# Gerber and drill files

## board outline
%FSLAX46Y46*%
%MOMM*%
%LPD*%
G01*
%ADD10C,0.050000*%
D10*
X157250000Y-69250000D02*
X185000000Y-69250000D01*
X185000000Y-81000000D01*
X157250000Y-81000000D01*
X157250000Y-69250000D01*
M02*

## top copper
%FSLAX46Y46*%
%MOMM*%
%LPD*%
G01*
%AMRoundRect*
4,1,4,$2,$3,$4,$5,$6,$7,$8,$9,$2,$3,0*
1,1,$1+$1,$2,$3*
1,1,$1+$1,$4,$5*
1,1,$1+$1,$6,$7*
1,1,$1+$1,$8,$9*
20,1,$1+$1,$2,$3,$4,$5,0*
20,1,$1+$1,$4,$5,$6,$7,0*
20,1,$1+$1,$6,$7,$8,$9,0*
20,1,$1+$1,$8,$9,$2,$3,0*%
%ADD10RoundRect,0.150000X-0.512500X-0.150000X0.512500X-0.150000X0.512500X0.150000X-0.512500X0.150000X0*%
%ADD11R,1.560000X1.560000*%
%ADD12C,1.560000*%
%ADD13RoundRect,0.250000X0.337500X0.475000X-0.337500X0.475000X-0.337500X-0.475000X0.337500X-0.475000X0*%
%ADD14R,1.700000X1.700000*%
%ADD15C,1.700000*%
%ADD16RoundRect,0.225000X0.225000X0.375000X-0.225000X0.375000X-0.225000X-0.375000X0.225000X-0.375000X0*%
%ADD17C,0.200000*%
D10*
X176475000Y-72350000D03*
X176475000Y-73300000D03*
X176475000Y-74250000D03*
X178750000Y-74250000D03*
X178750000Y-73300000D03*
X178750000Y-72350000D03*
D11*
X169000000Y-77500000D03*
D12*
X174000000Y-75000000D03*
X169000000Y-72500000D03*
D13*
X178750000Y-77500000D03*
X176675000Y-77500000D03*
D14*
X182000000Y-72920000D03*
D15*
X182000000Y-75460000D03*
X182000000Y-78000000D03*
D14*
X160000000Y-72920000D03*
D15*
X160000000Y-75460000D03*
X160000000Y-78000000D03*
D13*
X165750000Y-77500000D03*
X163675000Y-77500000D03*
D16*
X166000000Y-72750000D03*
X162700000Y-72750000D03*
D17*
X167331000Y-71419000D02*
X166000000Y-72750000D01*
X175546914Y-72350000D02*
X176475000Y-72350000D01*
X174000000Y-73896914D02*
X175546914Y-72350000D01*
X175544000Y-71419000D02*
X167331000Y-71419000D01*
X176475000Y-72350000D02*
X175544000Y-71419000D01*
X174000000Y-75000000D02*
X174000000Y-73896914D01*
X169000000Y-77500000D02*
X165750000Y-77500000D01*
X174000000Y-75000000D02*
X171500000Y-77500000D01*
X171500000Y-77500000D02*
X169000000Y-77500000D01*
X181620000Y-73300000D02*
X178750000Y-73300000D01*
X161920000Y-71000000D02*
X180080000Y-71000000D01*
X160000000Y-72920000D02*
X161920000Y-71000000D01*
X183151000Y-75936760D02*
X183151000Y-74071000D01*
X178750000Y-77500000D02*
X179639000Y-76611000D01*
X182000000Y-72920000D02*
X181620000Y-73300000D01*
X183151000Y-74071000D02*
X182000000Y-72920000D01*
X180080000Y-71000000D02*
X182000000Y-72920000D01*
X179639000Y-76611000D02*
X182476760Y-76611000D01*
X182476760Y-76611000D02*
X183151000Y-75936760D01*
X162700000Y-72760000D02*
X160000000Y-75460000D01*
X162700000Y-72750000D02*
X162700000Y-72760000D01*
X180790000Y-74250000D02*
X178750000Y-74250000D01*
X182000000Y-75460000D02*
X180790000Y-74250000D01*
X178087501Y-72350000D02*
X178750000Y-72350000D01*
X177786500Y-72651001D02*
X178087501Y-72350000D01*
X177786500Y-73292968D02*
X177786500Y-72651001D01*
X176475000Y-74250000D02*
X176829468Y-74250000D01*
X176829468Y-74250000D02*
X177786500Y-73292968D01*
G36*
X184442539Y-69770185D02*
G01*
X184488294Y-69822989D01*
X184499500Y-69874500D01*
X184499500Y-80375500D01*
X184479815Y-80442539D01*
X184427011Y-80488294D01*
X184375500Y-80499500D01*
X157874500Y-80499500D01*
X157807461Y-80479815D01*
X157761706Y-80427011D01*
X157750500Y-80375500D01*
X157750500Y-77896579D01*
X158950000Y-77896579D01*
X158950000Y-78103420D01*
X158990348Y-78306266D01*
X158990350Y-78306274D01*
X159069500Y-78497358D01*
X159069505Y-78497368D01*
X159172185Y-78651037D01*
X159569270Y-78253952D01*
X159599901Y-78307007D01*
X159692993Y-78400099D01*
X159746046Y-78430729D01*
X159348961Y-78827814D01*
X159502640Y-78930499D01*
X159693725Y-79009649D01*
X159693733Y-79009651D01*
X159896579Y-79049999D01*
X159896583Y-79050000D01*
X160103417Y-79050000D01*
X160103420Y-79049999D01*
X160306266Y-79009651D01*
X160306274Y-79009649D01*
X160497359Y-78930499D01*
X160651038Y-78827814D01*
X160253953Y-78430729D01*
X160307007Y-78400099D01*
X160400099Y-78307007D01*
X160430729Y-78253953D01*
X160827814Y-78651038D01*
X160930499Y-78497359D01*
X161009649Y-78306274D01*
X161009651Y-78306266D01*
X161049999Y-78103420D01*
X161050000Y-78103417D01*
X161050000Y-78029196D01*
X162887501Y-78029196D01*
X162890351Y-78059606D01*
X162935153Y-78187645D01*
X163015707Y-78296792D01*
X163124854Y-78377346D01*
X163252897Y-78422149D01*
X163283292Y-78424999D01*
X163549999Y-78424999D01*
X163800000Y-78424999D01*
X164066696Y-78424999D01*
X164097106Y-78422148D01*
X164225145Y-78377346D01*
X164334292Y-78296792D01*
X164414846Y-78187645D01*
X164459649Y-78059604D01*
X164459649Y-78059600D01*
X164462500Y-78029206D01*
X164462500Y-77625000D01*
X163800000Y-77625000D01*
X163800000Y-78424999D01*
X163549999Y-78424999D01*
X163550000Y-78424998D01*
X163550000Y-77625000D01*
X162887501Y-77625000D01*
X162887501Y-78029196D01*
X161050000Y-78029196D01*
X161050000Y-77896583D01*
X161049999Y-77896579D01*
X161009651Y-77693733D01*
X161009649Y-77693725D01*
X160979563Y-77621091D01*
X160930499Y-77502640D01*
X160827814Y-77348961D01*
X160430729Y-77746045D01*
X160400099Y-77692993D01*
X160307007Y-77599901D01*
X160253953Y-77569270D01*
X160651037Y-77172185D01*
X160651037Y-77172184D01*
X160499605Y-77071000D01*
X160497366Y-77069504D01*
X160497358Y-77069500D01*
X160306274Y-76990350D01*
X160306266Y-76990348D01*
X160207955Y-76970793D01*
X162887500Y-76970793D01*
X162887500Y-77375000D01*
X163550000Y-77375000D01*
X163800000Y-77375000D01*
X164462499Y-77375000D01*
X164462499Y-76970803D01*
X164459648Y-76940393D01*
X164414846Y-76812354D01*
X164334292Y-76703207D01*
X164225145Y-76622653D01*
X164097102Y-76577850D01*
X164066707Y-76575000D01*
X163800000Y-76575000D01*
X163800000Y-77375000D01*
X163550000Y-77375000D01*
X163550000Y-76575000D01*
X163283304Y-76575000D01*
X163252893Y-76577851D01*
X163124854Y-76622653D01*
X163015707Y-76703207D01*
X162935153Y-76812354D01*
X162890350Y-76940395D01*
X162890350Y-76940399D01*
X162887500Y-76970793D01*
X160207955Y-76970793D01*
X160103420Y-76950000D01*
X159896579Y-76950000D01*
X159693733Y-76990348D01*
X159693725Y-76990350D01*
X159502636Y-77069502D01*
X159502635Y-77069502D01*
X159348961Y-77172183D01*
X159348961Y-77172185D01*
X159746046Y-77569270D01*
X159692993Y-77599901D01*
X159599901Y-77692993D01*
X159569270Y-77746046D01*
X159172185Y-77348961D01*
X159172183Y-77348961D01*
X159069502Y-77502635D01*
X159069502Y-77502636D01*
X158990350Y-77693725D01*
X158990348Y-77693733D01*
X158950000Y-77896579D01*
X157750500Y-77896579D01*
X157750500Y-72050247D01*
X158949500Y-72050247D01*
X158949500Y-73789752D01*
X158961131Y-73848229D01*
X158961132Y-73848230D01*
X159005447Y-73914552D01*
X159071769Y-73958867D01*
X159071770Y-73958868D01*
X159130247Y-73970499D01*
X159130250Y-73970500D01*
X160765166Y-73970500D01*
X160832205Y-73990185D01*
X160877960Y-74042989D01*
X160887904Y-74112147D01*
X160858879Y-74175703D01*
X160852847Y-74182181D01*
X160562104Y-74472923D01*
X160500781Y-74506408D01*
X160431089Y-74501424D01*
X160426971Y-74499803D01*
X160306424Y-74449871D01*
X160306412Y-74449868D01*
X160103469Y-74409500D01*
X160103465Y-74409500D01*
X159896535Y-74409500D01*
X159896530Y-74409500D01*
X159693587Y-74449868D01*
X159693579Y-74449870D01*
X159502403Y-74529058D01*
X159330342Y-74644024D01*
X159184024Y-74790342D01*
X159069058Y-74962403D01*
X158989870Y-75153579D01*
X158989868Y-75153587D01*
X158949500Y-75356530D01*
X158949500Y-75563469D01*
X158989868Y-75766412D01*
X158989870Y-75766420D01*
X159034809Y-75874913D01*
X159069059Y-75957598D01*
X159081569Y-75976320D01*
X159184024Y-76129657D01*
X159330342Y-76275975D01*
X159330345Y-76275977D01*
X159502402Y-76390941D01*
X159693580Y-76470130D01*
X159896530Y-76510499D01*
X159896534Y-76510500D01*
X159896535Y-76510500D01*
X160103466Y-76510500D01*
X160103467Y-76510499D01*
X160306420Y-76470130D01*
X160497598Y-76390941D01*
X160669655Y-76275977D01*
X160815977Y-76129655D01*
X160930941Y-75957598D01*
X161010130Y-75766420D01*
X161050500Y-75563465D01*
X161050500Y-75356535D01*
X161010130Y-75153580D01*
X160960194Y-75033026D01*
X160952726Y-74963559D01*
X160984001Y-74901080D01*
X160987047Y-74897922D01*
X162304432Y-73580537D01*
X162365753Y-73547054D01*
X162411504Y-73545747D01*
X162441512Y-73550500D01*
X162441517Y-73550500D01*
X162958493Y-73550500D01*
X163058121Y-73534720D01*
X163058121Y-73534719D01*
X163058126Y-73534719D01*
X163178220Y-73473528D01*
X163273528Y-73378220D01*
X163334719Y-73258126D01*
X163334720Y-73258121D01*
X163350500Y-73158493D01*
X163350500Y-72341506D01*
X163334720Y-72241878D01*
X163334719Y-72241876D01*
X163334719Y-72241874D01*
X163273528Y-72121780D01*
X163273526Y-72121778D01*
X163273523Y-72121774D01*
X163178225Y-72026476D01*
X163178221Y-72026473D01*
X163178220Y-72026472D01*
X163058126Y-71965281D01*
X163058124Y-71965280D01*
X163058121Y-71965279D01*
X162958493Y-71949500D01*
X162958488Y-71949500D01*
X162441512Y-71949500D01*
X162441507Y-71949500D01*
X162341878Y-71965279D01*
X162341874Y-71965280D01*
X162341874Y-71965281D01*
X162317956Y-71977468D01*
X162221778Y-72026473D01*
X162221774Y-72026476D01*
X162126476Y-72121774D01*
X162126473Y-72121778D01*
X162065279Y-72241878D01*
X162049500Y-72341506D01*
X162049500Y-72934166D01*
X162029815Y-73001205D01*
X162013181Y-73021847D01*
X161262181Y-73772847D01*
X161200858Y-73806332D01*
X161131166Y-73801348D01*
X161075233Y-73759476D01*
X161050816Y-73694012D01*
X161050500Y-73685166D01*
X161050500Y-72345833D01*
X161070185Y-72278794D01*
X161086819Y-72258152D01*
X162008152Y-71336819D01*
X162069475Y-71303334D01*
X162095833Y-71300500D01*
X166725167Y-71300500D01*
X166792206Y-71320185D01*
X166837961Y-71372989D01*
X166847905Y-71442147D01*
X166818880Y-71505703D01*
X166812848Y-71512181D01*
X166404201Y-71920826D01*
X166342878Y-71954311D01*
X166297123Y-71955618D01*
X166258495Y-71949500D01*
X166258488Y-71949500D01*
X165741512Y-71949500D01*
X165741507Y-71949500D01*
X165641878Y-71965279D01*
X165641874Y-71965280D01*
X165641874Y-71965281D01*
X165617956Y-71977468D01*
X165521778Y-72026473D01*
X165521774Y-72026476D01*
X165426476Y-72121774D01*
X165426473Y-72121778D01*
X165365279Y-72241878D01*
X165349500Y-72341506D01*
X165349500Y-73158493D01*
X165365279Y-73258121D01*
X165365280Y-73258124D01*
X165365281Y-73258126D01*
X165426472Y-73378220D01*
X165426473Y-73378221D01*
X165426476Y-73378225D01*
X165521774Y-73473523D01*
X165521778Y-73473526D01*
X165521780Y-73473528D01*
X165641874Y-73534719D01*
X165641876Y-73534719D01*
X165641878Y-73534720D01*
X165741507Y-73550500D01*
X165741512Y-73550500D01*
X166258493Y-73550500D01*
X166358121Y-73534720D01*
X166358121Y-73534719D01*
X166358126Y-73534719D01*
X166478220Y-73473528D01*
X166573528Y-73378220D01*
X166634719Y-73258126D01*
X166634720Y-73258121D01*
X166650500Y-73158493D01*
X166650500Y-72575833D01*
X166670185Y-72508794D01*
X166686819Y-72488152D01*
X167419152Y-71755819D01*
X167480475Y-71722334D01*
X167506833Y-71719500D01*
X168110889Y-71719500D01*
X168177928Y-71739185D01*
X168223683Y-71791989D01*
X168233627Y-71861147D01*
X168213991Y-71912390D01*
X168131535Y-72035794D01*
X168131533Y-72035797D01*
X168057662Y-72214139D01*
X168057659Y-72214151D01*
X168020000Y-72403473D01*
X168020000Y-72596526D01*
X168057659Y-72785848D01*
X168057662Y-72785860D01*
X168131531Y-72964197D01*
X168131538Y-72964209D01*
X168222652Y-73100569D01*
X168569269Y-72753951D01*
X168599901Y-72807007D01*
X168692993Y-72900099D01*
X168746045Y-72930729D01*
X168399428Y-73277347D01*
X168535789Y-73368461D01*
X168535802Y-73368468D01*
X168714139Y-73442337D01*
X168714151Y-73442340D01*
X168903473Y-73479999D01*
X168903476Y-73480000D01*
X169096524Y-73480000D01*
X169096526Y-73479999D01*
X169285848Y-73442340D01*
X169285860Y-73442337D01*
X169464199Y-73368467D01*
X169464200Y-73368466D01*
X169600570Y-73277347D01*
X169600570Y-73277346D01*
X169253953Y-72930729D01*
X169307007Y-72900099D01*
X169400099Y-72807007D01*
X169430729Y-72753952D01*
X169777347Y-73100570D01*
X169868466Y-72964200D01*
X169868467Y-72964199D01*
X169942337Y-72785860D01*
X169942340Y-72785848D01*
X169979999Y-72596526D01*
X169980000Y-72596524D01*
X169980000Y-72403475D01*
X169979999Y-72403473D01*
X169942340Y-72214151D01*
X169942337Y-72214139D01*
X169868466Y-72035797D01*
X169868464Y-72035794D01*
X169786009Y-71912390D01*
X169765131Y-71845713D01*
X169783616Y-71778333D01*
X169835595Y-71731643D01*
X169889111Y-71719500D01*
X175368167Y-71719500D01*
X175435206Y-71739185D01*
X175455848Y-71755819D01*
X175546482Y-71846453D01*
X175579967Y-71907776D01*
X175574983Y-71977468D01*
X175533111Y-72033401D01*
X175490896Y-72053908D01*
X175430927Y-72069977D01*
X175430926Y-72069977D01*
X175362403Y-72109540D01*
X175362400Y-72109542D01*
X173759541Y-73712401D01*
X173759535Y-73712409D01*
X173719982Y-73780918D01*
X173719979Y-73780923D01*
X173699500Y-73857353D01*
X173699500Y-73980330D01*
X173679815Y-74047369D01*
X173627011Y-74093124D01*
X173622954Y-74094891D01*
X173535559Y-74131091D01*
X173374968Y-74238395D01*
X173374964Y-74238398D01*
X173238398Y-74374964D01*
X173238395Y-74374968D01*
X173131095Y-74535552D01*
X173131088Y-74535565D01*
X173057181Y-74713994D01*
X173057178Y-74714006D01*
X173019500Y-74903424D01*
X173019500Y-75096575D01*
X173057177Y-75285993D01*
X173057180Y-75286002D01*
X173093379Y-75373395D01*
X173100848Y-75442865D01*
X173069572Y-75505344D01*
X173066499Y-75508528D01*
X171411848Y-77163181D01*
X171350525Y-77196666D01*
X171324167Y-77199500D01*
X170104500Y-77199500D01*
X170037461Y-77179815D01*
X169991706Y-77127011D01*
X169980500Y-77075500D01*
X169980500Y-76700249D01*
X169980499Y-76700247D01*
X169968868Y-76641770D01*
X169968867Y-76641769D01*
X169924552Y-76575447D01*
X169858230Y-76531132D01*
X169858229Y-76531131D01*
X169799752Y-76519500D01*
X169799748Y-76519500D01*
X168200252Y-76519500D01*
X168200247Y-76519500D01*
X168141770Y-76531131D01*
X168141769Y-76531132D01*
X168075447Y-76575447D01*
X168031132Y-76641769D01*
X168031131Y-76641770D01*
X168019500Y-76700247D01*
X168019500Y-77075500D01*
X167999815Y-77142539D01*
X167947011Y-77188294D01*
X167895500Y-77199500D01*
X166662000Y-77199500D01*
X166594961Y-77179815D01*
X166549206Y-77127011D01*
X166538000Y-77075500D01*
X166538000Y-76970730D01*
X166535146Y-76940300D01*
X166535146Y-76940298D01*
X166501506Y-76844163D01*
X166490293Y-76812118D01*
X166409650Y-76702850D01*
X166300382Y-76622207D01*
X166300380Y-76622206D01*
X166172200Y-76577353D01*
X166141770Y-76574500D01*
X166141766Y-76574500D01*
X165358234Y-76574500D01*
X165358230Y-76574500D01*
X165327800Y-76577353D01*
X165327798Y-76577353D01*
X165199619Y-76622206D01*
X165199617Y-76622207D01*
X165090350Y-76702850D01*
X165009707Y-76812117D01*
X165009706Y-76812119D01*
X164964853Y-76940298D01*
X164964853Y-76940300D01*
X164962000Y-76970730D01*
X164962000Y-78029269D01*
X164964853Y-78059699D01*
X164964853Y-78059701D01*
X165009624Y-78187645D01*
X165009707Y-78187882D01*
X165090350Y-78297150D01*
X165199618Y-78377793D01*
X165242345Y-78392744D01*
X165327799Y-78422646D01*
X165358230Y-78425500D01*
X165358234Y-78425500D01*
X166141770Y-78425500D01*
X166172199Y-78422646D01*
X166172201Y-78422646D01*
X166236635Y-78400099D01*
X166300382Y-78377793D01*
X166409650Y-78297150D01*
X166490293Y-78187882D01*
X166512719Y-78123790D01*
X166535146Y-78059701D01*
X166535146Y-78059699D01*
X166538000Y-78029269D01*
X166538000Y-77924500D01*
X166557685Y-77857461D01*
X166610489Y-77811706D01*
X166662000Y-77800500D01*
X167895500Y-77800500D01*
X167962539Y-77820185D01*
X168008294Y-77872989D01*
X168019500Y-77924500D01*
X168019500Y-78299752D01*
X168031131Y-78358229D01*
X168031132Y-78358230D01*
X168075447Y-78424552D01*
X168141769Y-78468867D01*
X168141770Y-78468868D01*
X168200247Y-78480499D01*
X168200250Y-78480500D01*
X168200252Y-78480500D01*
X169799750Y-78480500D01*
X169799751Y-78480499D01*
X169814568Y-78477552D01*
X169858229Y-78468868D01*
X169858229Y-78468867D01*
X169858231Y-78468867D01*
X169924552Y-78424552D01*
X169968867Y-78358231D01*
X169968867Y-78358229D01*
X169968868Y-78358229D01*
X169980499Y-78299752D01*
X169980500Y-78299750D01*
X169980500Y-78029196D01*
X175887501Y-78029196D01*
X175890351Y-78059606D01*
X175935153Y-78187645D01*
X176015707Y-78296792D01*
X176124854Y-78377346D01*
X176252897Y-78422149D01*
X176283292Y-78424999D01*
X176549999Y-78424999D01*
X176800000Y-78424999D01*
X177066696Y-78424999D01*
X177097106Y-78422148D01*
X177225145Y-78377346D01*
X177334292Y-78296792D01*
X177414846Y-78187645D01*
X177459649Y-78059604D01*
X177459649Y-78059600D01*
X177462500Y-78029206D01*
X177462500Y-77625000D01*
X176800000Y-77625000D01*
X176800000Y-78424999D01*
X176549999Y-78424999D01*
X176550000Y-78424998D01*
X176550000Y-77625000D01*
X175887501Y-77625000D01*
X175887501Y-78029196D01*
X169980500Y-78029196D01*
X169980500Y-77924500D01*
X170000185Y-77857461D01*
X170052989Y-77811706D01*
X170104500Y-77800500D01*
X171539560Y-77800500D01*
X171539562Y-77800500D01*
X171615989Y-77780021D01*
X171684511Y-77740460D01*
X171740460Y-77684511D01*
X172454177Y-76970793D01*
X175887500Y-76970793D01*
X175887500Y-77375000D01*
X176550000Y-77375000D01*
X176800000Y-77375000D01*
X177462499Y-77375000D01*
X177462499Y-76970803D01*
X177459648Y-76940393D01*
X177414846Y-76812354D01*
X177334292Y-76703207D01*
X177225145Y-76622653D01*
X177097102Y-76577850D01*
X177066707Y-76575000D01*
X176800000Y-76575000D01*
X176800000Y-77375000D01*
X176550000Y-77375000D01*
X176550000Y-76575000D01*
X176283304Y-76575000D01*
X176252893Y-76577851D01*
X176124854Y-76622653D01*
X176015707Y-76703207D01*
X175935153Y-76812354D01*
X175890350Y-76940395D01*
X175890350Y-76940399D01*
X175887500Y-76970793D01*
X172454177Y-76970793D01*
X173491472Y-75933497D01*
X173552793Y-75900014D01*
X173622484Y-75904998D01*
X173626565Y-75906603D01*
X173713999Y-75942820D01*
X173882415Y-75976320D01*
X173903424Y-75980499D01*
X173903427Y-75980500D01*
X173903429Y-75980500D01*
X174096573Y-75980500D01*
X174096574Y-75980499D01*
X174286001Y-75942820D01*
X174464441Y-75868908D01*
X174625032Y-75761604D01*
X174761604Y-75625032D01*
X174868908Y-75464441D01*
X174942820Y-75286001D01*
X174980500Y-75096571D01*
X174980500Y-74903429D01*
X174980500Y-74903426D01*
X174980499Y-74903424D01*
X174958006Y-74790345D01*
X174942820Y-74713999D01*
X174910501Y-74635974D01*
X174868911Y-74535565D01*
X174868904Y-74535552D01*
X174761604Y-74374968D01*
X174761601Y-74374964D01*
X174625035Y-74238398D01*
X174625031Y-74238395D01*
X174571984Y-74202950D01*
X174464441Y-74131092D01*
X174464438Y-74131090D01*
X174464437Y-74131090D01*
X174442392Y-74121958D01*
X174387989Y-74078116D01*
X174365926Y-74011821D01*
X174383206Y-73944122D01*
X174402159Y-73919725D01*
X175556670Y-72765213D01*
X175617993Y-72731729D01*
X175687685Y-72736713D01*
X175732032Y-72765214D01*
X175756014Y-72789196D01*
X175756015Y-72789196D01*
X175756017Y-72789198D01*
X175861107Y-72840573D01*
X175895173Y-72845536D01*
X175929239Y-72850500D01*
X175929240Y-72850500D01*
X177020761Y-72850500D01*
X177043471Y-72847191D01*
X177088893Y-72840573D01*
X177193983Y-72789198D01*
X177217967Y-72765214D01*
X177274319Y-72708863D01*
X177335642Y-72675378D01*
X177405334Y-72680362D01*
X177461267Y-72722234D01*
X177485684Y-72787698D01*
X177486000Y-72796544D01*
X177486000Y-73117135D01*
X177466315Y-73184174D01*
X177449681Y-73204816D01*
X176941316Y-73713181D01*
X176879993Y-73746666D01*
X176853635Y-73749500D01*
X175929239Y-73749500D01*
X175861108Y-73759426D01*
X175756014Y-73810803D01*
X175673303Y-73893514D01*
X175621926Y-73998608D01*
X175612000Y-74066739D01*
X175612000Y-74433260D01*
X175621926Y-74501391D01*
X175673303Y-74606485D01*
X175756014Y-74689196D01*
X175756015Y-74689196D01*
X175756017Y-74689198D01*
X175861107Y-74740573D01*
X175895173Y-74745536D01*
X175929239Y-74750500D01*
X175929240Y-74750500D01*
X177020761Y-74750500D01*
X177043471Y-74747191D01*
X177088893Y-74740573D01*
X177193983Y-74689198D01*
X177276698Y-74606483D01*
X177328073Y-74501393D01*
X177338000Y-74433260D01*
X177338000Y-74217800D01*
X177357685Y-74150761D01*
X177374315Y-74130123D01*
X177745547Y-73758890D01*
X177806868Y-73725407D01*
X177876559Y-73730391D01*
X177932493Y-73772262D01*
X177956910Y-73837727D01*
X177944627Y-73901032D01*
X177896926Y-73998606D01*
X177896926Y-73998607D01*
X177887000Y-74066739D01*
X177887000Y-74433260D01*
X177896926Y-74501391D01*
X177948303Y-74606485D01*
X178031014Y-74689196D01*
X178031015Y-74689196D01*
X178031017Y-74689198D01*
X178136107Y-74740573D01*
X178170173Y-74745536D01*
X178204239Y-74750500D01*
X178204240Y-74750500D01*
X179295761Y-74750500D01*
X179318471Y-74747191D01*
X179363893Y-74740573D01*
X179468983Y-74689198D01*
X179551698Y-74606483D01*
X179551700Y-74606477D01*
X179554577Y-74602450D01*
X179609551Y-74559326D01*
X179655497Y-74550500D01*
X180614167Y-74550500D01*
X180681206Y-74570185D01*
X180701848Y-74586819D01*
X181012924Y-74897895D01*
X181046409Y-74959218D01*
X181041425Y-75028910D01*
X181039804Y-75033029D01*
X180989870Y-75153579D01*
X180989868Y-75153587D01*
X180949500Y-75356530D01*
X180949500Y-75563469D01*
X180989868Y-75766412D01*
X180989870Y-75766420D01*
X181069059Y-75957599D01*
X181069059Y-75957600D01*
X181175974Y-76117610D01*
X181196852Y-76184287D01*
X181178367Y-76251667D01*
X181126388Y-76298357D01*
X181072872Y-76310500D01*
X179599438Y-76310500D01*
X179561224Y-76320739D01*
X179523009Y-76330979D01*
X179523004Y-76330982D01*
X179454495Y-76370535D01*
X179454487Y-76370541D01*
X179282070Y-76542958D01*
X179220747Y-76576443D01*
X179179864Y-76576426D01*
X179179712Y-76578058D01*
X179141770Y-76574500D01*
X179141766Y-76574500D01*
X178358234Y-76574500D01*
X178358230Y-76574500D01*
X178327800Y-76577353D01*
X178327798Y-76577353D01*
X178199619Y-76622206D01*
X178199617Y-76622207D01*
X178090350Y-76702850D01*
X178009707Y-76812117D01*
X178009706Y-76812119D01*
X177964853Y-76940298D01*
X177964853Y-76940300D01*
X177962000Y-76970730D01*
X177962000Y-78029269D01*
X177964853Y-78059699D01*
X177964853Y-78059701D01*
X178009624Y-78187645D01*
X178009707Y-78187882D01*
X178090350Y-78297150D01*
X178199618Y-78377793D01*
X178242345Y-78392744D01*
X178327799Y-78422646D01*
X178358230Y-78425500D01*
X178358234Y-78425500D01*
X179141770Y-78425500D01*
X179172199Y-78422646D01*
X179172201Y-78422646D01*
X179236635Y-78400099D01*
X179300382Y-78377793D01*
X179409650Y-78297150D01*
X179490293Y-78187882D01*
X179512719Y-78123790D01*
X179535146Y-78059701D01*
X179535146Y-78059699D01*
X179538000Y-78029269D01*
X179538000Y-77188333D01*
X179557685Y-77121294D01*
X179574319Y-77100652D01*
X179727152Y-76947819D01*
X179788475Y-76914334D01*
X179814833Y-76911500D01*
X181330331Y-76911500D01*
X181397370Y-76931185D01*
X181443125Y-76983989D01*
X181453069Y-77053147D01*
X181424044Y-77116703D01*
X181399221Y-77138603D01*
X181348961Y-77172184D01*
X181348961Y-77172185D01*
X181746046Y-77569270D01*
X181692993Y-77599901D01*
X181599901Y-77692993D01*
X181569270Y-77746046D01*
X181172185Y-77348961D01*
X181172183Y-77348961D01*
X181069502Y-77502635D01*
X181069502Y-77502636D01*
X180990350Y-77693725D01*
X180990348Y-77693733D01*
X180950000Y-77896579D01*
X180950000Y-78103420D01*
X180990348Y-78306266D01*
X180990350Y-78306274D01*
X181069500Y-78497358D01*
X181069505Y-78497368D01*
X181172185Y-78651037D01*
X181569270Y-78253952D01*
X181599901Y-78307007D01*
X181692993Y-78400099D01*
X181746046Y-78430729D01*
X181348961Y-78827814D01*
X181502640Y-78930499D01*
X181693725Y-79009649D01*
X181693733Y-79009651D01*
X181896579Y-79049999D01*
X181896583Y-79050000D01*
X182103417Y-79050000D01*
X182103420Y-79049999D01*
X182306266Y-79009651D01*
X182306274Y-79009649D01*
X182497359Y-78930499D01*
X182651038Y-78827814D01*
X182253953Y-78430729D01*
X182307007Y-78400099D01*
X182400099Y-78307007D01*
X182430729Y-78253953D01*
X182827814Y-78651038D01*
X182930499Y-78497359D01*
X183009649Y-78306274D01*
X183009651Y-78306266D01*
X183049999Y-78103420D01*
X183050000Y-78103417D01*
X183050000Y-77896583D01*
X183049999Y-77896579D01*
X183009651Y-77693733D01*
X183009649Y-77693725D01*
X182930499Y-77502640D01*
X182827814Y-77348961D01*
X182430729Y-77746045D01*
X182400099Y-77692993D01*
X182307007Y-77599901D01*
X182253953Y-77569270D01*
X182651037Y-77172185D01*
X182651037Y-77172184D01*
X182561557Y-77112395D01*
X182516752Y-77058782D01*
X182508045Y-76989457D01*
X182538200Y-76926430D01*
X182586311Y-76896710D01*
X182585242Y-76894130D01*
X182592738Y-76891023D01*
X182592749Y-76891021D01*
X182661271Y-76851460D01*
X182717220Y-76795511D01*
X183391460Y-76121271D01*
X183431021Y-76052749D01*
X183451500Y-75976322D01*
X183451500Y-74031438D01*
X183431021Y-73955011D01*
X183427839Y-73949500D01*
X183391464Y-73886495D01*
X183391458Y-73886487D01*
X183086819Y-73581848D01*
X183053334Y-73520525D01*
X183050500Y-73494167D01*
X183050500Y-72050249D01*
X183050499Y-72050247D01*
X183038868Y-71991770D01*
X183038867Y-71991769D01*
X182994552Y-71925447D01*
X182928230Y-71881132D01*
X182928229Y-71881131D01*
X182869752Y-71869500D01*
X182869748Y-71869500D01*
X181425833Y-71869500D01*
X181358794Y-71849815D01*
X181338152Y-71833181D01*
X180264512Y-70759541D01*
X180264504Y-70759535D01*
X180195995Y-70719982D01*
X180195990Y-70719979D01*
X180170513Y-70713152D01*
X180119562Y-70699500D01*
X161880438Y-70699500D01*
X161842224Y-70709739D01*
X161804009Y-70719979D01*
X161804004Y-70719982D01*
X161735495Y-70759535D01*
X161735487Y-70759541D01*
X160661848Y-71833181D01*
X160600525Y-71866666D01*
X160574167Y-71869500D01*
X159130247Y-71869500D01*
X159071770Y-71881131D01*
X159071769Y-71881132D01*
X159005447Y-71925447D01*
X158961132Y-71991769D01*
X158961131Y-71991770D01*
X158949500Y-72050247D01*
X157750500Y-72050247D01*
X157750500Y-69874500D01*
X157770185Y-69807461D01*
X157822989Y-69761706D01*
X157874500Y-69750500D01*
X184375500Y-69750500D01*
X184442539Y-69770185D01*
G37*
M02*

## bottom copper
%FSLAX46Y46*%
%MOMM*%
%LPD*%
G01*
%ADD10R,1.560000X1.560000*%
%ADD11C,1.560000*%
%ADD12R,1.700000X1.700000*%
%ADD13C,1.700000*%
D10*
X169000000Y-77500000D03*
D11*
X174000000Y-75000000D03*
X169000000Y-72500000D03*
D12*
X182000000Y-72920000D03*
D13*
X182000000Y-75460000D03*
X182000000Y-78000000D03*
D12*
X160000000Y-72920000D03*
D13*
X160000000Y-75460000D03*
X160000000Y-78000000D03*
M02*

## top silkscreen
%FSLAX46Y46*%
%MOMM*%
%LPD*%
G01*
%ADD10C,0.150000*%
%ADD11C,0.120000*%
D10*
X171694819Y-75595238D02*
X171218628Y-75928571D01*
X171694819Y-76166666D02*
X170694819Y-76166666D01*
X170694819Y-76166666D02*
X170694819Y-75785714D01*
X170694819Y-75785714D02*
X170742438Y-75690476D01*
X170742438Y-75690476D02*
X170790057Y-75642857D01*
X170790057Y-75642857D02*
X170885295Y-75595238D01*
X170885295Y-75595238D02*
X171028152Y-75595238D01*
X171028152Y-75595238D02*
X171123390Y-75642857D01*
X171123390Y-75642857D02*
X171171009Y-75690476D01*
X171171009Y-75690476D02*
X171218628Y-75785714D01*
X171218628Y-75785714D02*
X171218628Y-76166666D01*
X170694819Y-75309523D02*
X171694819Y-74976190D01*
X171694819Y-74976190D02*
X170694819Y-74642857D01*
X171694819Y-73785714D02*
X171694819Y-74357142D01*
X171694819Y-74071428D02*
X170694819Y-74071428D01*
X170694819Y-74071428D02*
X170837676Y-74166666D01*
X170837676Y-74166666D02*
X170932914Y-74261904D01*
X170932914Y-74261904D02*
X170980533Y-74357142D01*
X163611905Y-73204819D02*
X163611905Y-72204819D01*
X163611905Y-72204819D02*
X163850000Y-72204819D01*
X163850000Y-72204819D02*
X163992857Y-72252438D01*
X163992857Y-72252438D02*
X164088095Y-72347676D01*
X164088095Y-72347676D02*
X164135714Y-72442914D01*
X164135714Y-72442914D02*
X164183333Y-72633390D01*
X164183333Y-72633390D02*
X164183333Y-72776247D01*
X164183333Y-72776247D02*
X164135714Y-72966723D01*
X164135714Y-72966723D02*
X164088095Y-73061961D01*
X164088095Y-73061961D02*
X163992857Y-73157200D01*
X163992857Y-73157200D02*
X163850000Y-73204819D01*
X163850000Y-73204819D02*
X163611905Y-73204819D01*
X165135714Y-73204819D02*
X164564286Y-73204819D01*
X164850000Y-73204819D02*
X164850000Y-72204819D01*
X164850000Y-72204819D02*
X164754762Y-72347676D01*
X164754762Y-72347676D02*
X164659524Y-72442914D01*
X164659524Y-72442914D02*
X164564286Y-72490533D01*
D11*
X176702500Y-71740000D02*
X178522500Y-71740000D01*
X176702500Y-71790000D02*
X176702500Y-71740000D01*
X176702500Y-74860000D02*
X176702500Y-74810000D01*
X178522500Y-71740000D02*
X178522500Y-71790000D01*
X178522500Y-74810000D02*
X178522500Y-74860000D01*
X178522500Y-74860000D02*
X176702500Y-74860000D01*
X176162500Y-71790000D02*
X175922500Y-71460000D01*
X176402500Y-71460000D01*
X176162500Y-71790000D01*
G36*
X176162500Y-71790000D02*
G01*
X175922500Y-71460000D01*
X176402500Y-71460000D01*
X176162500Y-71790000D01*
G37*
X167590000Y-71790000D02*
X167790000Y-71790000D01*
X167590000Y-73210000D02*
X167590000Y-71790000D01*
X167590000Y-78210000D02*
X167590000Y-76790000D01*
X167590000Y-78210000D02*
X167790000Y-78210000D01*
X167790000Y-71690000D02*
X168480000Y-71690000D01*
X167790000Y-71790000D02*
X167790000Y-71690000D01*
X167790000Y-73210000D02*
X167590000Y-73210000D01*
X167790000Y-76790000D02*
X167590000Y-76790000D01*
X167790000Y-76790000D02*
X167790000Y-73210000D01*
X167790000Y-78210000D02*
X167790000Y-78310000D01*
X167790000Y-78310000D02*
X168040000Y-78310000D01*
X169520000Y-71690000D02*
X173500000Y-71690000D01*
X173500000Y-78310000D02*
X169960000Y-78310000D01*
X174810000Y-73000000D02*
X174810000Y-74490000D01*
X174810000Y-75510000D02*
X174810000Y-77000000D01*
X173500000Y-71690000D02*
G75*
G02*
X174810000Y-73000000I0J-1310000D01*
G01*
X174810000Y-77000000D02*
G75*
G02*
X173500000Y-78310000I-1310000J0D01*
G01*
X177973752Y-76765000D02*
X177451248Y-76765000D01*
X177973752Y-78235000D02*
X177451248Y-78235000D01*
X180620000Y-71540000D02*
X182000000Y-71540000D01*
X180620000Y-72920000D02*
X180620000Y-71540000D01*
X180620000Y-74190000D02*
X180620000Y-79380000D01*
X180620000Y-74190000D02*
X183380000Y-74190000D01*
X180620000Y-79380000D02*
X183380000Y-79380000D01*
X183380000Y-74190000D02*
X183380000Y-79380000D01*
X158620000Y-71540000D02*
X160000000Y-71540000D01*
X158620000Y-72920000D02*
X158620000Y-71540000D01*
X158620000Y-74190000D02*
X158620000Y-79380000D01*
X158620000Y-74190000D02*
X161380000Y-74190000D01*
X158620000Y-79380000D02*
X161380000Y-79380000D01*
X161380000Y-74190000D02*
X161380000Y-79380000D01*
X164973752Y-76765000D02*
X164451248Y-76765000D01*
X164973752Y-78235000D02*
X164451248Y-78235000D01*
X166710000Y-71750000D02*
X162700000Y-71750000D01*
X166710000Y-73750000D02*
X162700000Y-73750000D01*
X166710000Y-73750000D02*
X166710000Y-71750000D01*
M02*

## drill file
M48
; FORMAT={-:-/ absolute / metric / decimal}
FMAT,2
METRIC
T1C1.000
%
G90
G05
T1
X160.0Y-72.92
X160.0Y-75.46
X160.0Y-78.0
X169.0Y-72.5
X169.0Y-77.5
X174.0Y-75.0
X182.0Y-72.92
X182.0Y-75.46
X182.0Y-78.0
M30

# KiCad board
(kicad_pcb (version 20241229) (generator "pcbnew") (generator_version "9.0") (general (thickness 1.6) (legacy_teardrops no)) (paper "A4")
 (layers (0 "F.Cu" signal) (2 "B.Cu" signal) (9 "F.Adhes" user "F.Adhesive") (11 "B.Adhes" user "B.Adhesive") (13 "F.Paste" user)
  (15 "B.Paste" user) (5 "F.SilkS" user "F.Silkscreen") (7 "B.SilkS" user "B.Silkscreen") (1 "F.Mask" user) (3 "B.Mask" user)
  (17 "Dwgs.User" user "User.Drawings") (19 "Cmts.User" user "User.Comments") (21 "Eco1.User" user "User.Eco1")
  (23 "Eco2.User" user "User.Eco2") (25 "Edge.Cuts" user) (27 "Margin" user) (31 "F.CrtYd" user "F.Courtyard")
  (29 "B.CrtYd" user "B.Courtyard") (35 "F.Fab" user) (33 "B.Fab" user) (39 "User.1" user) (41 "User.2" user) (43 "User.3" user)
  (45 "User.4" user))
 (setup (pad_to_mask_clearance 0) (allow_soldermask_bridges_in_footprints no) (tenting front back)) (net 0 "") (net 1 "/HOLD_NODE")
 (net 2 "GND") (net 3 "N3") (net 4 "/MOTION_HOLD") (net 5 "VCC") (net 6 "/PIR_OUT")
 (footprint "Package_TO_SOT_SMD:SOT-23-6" (layer "F.Cu") (at 177.6125 73.3)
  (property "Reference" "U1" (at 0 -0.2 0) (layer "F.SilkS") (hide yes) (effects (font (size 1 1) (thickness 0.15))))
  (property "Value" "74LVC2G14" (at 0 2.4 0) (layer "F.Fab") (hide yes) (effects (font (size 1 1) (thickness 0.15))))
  (fp_line (start -0.91 -1.56) (end 0.91 -1.56) (stroke (width 0.12) (type solid)) (layer "F.SilkS"))
  (fp_line (start -0.91 -1.51) (end -0.91 -1.56) (stroke (width 0.12) (type solid)) (layer "F.SilkS"))
  (fp_line (start -0.91 1.56) (end -0.91 1.51) (stroke (width 0.12) (type solid)) (layer "F.SilkS"))
  (fp_line (start 0.91 -1.56) (end 0.91 -1.51) (stroke (width 0.12) (type solid)) (layer "F.SilkS"))
  (fp_line (start 0.91 1.51) (end 0.91 1.56) (stroke (width 0.12) (type solid)) (layer "F.SilkS"))
  (fp_line (start 0.91 1.56) (end -0.91 1.56) (stroke (width 0.12) (type solid)) (layer "F.SilkS"))
  (fp_poly (pts (xy -1.45 -1.51) (xy -1.69 -1.84) (xy -1.21 -1.84)) (stroke (width 0.12) (type solid)) (fill yes) (layer "F.SilkS"))
  (pad "1" smd roundrect (at -1.1375 -0.95) (size 1.325 0.6) (layers "F.Cu" "F.Mask" "F.Paste") (roundrect_rratio 0.25) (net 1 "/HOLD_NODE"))
  (pad "2" smd roundrect (at -1.1375 0) (size 1.325 0.6) (layers "F.Cu" "F.Mask" "F.Paste") (roundrect_rratio 0.25) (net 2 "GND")
   (zone_connect 2))
  (pad "3" smd roundrect (at -1.1375 0.95) (size 1.325 0.6) (layers "F.Cu" "F.Mask" "F.Paste") (roundrect_rratio 0.25) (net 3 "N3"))
  (pad "4" smd roundrect (at 1.1375 0.95) (size 1.325 0.6) (layers "F.Cu" "F.Mask" "F.Paste") (roundrect_rratio 0.25) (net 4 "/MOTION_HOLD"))
  (pad "5" smd roundrect (at 1.1375 0) (size 1.325 0.6) (layers "F.Cu" "F.Mask" "F.Paste") (roundrect_rratio 0.25) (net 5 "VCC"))
  (pad "6" smd roundrect (at 1.1375 -0.95) (size 1.325 0.6) (layers "F.Cu" "F.Mask" "F.Paste") (roundrect_rratio 0.25) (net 3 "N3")))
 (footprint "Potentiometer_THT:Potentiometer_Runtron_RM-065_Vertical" (layer "F.Cu") (at 169 77.5 90)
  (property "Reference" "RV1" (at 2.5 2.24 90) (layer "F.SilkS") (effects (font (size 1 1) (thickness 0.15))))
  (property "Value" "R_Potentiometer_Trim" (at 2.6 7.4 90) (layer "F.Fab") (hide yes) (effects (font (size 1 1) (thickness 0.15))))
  (fp_line (start 5.71 -1.41) (end 5.71 -1.21) (stroke (width 0.12) (type solid)) (layer "F.SilkS"))
  (fp_line (start 4.29 -1.41) (end 5.71 -1.41) (stroke (width 0.12) (type solid)) (layer "F.SilkS"))
  (fp_line (start -0.71 -1.41) (end 0.71 -1.41) (stroke (width 0.12) (type solid)) (layer "F.SilkS"))
  (fp_line (start -0.71 -1.41) (end -0.71 -1.21) (stroke (width 0.12) (type solid)) (layer "F.SilkS"))
  (fp_line (start 5.81 -1.21) (end 5.81 -0.52) (stroke (width 0.12) (type solid)) (layer "F.SilkS"))
  (fp_line (start 5.71 -1.21) (end 5.81 -1.21) (stroke (width 0.12) (type solid)) (layer "F.SilkS"))
  (fp_line (start 4.29 -1.21) (end 4.29 -1.41) (stroke (width 0.12) (type solid)) (layer "F.SilkS"))
  (fp_line (start 0.71 -1.21) (end 0.71 -1.41) (stroke (width 0.12) (type solid)) (layer "F.SilkS"))
  (fp_line (start 0.71 -1.21) (end 4.29 -1.21) (stroke (width 0.12) (type solid)) (layer "F.SilkS"))
  (fp_line (start -0.71 -1.21) (end -0.81 -1.21) (stroke (width 0.12) (type solid)) (layer "F.SilkS"))
  (fp_line (start -0.81 -1.21) (end -0.81 -0.96) (stroke (width 0.12) (type solid)) (layer "F.SilkS"))
  (fp_line (start 5.81 0.52) (end 5.81 4.5) (stroke (width 0.12) (type solid)) (layer "F.SilkS"))
  (fp_line (start -0.81 4.5) (end -0.81 0.96) (stroke (width 0.12) (type solid)) (layer "F.SilkS"))
  (fp_line (start 4.5 5.81) (end 3.01 5.81) (stroke (width 0.12) (type solid)) (layer "F.SilkS"))
  (fp_line (start 1.99 5.81) (end 0.5 5.81) (stroke (width 0.12) (type solid)) (layer "F.SilkS"))
  (fp_arc (start 5.81 4.5) (mid 5.42631 5.42631) (end 4.5 5.81) (stroke (width 0.12) (type solid)) (layer "F.SilkS"))
  (fp_arc (start 0.5 5.81) (mid -0.42631 5.42631) (end -0.81 4.5) (stroke (width 0.12) (type solid)) (layer "F.SilkS"))
  (pad "1" thru_hole rect (at 0 0 90) (size 1.56 1.56) (drill 1) (layers "*.Cu" "*.Mask") (remove_unused_layers no) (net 1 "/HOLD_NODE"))
  (pad "2" thru_hole circle (at 2.5 5 90) (size 1.56 1.56) (drill 1) (layers "*.Cu" "*.Mask") (remove_unused_layers no) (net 1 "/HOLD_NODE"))
  (pad "3" thru_hole circle (at 5 0 90) (size 1.56 1.56) (drill 1) (layers "*.Cu" "*.Mask") (remove_unused_layers no) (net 2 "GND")))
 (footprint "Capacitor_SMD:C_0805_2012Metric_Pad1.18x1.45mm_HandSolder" (layer "F.Cu") (at 177.7125 77.5 180)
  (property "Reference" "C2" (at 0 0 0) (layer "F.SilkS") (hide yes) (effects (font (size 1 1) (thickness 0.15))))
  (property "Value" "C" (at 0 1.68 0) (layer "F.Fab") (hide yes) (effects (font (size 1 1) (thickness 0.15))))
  (fp_line (start -0.261252 0.735) (end 0.261252 0.735) (stroke (width 0.12) (type solid)) (layer "F.SilkS"))
  (fp_line (start -0.261252 -0.735) (end 0.261252 -0.735) (stroke (width 0.12) (type solid)) (layer "F.SilkS"))
  (pad "1" smd roundrect (at -1.0375 0 180) (size 1.175 1.45) (layers "F.Cu" "F.Mask" "F.Paste") (roundrect_rratio 0.212766) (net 5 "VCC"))
  (pad "2" smd roundrect (at 1.0375 0 180) (size 1.175 1.45) (layers "F.Cu" "F.Mask" "F.Paste") (roundrect_rratio 0.212766) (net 2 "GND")))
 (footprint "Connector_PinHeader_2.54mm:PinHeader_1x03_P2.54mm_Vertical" (layer "F.Cu") (at 182 72.92)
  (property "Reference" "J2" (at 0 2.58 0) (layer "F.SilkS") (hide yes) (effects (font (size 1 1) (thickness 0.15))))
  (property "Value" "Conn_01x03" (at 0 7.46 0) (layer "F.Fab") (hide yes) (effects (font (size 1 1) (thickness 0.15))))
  (fp_line (start -1.38 -1.38) (end 0 -1.38) (stroke (width 0.12) (type solid)) (layer "F.SilkS"))
  (fp_line (start -1.38 0) (end -1.38 -1.38) (stroke (width 0.12) (type solid)) (layer "F.SilkS"))
  (fp_line (start -1.38 1.27) (end -1.38 6.46) (stroke (width 0.12) (type solid)) (layer "F.SilkS"))
  (fp_line (start -1.38 1.27) (end 1.38 1.27) (stroke (width 0.12) (type solid)) (layer "F.SilkS"))
  (fp_line (start -1.38 6.46) (end 1.38 6.46) (stroke (width 0.12) (type solid)) (layer "F.SilkS"))
  (fp_line (start 1.38 1.27) (end 1.38 6.46) (stroke (width 0.12) (type solid)) (layer "F.SilkS"))
  (pad "1" thru_hole rect (at 0 0) (size 1.7 1.7) (drill 1) (layers "*.Cu" "*.Mask") (remove_unused_layers no) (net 5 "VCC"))
  (pad "2" thru_hole circle (at 0 2.54) (size 1.7 1.7) (drill 1) (layers "*.Cu" "*.Mask") (remove_unused_layers no) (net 4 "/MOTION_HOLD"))
  (pad "3" thru_hole circle (at 0 5.08) (size 1.7 1.7) (drill 1) (layers "*.Cu" "*.Mask") (remove_unused_layers no) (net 2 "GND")))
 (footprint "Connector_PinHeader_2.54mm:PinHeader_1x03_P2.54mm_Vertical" (layer "F.Cu") (at 160 72.92)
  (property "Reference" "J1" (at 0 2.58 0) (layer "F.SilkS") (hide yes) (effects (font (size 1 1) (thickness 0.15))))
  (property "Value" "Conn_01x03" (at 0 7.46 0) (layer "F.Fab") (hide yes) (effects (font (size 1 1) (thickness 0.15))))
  (fp_line (start -1.38 -1.38) (end 0 -1.38) (stroke (width 0.12) (type solid)) (layer "F.SilkS"))
  (fp_line (start -1.38 0) (end -1.38 -1.38) (stroke (width 0.12) (type solid)) (layer "F.SilkS"))
  (fp_line (start -1.38 1.27) (end -1.38 6.46) (stroke (width 0.12) (type solid)) (layer "F.SilkS"))
  (fp_line (start -1.38 1.27) (end 1.38 1.27) (stroke (width 0.12) (type solid)) (layer "F.SilkS"))
  (fp_line (start -1.38 6.46) (end 1.38 6.46) (stroke (width 0.12) (type solid)) (layer "F.SilkS"))
  (fp_line (start 1.38 1.27) (end 1.38 6.46) (stroke (width 0.12) (type solid)) (layer "F.SilkS"))
  (pad "1" thru_hole rect (at 0 0) (size 1.7 1.7) (drill 1) (layers "*.Cu" "*.Mask") (remove_unused_layers no) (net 5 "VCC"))
  (pad "2" thru_hole circle (at 0 2.54) (size 1.7 1.7) (drill 1) (layers "*.Cu" "*.Mask") (remove_unused_layers no) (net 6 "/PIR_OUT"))
  (pad "3" thru_hole circle (at 0 5.08) (size 1.7 1.7) (drill 1) (layers "*.Cu" "*.Mask") (remove_unused_layers no) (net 2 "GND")))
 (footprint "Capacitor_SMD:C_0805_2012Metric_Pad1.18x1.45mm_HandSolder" (layer "F.Cu") (at 164.7125 77.5 180)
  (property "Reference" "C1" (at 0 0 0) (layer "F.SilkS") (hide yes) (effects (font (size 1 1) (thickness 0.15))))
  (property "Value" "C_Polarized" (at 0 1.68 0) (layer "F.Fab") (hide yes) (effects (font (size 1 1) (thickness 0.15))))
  (fp_line (start -0.261252 0.735) (end 0.261252 0.735) (stroke (width 0.12) (type solid)) (layer "F.SilkS"))
  (fp_line (start -0.261252 -0.735) (end 0.261252 -0.735) (stroke (width 0.12) (type solid)) (layer "F.SilkS"))
  (pad "1" smd roundrect (at -1.0375 0 180) (size 1.175 1.45) (layers "F.Cu" "F.Mask" "F.Paste") (roundrect_rratio 0.212766)
   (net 1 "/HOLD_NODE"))
  (pad "2" smd roundrect (at 1.0375 0 180) (size 1.175 1.45) (layers "F.Cu" "F.Mask" "F.Paste") (roundrect_rratio 0.212766) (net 2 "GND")))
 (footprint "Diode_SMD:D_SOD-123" (layer "F.Cu") (at 164.35 72.75 180)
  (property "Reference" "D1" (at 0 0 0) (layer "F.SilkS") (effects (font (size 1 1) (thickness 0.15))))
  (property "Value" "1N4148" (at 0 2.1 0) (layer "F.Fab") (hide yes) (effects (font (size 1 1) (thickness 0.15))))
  (fp_line (start -2.36 1) (end 1.65 1) (stroke (width 0.12) (type solid)) (layer "F.SilkS"))
  (fp_line (start -2.36 -1) (end 1.65 -1) (stroke (width 0.12) (type solid)) (layer "F.SilkS"))
  (fp_line (start -2.36 -1) (end -2.36 1) (stroke (width 0.12) (type solid)) (layer "F.SilkS"))
  (pad "1" smd roundrect (at -1.65 0 180) (size 0.9 1.2) (layers "F.Cu" "F.Mask" "F.Paste") (roundrect_rratio 0.25) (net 1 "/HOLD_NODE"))
  (pad "2" smd roundrect (at 1.65 0 180) (size 0.9 1.2) (layers "F.Cu" "F.Mask" "F.Paste") (roundrect_rratio 0.25) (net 6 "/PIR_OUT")))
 (gr_rect (start 157.25 69.25) (end 185 81) (stroke (width 0.05) (type default)) (fill no) (layer "Edge.Cuts"))
 (segment (start 167.331 71.419) (end 166 72.75) (width 0.2) (layer "F.Cu") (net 1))
 (segment (start 175.546914 72.35) (end 176.475 72.35) (width 0.2) (layer "F.Cu") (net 1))
 (segment (start 174 73.896914) (end 175.546914 72.35) (width 0.2) (layer "F.Cu") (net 1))
 (segment (start 175.544 71.419) (end 167.331 71.419) (width 0.2) (layer "F.Cu") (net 1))
 (segment (start 176.475 72.35) (end 175.544 71.419) (width 0.2) (layer "F.Cu") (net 1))
 (segment (start 174 75) (end 174 73.896914) (width 0.2) (layer "F.Cu") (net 1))
 (segment (start 169 77.5) (end 165.75 77.5) (width 0.2) (layer "F.Cu") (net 1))
 (segment (start 174 75) (end 171.5 77.5) (width 0.2) (layer "F.Cu") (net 1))
 (segment (start 171.5 77.5) (end 169 77.5) (width 0.2) (layer "F.Cu") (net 1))
 (segment (start 181.62 73.3) (end 178.75 73.3) (width 0.2) (layer "F.Cu") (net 5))
 (segment (start 161.92 71) (end 180.08 71) (width 0.2) (layer "F.Cu") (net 5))
 (segment (start 160 72.92) (end 161.92 71) (width 0.2) (layer "F.Cu") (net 5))
 (segment (start 183.151 75.93676) (end 183.151 74.071) (width 0.2) (layer "F.Cu") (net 5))
 (segment (start 178.75 77.5) (end 179.639 76.611) (width 0.2) (layer "F.Cu") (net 5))
 (segment (start 182 72.92) (end 181.62 73.3) (width 0.2) (layer "F.Cu") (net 5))
 (segment (start 183.151 74.071) (end 182 72.92) (width 0.2) (layer "F.Cu") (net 5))
 (segment (start 180.08 71) (end 182 72.92) (width 0.2) (layer "F.Cu") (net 5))
 (segment (start 179.639 76.611) (end 182.47676 76.611) (width 0.2) (layer "F.Cu") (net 5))
 (segment (start 182.47676 76.611) (end 183.151 75.93676) (width 0.2) (layer "F.Cu") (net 5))
 (segment (start 162.7 72.76) (end 160 75.46) (width 0.2) (layer "F.Cu") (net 6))
 (segment (start 162.7 72.75) (end 162.7 72.76) (width 0.2) (layer "F.Cu") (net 6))
 (segment (start 180.79 74.25) (end 178.75 74.25) (width 0.2) (layer "F.Cu") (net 4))
 (segment (start 182 75.46) (end 180.79 74.25) (width 0.2) (layer "F.Cu") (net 4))
 (segment (start 178.087501 72.35) (end 178.75 72.35) (width 0.2) (layer "F.Cu") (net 3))
 (segment (start 177.7865 72.651001) (end 178.087501 72.35) (width 0.2) (layer "F.Cu") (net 3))
 (segment (start 177.7865 73.292968) (end 177.7865 72.651001) (width 0.2) (layer "F.Cu") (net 3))
 (segment (start 176.475 74.25) (end 176.829468 74.25) (width 0.2) (layer "F.Cu") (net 3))
 (segment (start 176.829468 74.25) (end 177.7865 73.292968) (width 0.2) (layer "F.Cu") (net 3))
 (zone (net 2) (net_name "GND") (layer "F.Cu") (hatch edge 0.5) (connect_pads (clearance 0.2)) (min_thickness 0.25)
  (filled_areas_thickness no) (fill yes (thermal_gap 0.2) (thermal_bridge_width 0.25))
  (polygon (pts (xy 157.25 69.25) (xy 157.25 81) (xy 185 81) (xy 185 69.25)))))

